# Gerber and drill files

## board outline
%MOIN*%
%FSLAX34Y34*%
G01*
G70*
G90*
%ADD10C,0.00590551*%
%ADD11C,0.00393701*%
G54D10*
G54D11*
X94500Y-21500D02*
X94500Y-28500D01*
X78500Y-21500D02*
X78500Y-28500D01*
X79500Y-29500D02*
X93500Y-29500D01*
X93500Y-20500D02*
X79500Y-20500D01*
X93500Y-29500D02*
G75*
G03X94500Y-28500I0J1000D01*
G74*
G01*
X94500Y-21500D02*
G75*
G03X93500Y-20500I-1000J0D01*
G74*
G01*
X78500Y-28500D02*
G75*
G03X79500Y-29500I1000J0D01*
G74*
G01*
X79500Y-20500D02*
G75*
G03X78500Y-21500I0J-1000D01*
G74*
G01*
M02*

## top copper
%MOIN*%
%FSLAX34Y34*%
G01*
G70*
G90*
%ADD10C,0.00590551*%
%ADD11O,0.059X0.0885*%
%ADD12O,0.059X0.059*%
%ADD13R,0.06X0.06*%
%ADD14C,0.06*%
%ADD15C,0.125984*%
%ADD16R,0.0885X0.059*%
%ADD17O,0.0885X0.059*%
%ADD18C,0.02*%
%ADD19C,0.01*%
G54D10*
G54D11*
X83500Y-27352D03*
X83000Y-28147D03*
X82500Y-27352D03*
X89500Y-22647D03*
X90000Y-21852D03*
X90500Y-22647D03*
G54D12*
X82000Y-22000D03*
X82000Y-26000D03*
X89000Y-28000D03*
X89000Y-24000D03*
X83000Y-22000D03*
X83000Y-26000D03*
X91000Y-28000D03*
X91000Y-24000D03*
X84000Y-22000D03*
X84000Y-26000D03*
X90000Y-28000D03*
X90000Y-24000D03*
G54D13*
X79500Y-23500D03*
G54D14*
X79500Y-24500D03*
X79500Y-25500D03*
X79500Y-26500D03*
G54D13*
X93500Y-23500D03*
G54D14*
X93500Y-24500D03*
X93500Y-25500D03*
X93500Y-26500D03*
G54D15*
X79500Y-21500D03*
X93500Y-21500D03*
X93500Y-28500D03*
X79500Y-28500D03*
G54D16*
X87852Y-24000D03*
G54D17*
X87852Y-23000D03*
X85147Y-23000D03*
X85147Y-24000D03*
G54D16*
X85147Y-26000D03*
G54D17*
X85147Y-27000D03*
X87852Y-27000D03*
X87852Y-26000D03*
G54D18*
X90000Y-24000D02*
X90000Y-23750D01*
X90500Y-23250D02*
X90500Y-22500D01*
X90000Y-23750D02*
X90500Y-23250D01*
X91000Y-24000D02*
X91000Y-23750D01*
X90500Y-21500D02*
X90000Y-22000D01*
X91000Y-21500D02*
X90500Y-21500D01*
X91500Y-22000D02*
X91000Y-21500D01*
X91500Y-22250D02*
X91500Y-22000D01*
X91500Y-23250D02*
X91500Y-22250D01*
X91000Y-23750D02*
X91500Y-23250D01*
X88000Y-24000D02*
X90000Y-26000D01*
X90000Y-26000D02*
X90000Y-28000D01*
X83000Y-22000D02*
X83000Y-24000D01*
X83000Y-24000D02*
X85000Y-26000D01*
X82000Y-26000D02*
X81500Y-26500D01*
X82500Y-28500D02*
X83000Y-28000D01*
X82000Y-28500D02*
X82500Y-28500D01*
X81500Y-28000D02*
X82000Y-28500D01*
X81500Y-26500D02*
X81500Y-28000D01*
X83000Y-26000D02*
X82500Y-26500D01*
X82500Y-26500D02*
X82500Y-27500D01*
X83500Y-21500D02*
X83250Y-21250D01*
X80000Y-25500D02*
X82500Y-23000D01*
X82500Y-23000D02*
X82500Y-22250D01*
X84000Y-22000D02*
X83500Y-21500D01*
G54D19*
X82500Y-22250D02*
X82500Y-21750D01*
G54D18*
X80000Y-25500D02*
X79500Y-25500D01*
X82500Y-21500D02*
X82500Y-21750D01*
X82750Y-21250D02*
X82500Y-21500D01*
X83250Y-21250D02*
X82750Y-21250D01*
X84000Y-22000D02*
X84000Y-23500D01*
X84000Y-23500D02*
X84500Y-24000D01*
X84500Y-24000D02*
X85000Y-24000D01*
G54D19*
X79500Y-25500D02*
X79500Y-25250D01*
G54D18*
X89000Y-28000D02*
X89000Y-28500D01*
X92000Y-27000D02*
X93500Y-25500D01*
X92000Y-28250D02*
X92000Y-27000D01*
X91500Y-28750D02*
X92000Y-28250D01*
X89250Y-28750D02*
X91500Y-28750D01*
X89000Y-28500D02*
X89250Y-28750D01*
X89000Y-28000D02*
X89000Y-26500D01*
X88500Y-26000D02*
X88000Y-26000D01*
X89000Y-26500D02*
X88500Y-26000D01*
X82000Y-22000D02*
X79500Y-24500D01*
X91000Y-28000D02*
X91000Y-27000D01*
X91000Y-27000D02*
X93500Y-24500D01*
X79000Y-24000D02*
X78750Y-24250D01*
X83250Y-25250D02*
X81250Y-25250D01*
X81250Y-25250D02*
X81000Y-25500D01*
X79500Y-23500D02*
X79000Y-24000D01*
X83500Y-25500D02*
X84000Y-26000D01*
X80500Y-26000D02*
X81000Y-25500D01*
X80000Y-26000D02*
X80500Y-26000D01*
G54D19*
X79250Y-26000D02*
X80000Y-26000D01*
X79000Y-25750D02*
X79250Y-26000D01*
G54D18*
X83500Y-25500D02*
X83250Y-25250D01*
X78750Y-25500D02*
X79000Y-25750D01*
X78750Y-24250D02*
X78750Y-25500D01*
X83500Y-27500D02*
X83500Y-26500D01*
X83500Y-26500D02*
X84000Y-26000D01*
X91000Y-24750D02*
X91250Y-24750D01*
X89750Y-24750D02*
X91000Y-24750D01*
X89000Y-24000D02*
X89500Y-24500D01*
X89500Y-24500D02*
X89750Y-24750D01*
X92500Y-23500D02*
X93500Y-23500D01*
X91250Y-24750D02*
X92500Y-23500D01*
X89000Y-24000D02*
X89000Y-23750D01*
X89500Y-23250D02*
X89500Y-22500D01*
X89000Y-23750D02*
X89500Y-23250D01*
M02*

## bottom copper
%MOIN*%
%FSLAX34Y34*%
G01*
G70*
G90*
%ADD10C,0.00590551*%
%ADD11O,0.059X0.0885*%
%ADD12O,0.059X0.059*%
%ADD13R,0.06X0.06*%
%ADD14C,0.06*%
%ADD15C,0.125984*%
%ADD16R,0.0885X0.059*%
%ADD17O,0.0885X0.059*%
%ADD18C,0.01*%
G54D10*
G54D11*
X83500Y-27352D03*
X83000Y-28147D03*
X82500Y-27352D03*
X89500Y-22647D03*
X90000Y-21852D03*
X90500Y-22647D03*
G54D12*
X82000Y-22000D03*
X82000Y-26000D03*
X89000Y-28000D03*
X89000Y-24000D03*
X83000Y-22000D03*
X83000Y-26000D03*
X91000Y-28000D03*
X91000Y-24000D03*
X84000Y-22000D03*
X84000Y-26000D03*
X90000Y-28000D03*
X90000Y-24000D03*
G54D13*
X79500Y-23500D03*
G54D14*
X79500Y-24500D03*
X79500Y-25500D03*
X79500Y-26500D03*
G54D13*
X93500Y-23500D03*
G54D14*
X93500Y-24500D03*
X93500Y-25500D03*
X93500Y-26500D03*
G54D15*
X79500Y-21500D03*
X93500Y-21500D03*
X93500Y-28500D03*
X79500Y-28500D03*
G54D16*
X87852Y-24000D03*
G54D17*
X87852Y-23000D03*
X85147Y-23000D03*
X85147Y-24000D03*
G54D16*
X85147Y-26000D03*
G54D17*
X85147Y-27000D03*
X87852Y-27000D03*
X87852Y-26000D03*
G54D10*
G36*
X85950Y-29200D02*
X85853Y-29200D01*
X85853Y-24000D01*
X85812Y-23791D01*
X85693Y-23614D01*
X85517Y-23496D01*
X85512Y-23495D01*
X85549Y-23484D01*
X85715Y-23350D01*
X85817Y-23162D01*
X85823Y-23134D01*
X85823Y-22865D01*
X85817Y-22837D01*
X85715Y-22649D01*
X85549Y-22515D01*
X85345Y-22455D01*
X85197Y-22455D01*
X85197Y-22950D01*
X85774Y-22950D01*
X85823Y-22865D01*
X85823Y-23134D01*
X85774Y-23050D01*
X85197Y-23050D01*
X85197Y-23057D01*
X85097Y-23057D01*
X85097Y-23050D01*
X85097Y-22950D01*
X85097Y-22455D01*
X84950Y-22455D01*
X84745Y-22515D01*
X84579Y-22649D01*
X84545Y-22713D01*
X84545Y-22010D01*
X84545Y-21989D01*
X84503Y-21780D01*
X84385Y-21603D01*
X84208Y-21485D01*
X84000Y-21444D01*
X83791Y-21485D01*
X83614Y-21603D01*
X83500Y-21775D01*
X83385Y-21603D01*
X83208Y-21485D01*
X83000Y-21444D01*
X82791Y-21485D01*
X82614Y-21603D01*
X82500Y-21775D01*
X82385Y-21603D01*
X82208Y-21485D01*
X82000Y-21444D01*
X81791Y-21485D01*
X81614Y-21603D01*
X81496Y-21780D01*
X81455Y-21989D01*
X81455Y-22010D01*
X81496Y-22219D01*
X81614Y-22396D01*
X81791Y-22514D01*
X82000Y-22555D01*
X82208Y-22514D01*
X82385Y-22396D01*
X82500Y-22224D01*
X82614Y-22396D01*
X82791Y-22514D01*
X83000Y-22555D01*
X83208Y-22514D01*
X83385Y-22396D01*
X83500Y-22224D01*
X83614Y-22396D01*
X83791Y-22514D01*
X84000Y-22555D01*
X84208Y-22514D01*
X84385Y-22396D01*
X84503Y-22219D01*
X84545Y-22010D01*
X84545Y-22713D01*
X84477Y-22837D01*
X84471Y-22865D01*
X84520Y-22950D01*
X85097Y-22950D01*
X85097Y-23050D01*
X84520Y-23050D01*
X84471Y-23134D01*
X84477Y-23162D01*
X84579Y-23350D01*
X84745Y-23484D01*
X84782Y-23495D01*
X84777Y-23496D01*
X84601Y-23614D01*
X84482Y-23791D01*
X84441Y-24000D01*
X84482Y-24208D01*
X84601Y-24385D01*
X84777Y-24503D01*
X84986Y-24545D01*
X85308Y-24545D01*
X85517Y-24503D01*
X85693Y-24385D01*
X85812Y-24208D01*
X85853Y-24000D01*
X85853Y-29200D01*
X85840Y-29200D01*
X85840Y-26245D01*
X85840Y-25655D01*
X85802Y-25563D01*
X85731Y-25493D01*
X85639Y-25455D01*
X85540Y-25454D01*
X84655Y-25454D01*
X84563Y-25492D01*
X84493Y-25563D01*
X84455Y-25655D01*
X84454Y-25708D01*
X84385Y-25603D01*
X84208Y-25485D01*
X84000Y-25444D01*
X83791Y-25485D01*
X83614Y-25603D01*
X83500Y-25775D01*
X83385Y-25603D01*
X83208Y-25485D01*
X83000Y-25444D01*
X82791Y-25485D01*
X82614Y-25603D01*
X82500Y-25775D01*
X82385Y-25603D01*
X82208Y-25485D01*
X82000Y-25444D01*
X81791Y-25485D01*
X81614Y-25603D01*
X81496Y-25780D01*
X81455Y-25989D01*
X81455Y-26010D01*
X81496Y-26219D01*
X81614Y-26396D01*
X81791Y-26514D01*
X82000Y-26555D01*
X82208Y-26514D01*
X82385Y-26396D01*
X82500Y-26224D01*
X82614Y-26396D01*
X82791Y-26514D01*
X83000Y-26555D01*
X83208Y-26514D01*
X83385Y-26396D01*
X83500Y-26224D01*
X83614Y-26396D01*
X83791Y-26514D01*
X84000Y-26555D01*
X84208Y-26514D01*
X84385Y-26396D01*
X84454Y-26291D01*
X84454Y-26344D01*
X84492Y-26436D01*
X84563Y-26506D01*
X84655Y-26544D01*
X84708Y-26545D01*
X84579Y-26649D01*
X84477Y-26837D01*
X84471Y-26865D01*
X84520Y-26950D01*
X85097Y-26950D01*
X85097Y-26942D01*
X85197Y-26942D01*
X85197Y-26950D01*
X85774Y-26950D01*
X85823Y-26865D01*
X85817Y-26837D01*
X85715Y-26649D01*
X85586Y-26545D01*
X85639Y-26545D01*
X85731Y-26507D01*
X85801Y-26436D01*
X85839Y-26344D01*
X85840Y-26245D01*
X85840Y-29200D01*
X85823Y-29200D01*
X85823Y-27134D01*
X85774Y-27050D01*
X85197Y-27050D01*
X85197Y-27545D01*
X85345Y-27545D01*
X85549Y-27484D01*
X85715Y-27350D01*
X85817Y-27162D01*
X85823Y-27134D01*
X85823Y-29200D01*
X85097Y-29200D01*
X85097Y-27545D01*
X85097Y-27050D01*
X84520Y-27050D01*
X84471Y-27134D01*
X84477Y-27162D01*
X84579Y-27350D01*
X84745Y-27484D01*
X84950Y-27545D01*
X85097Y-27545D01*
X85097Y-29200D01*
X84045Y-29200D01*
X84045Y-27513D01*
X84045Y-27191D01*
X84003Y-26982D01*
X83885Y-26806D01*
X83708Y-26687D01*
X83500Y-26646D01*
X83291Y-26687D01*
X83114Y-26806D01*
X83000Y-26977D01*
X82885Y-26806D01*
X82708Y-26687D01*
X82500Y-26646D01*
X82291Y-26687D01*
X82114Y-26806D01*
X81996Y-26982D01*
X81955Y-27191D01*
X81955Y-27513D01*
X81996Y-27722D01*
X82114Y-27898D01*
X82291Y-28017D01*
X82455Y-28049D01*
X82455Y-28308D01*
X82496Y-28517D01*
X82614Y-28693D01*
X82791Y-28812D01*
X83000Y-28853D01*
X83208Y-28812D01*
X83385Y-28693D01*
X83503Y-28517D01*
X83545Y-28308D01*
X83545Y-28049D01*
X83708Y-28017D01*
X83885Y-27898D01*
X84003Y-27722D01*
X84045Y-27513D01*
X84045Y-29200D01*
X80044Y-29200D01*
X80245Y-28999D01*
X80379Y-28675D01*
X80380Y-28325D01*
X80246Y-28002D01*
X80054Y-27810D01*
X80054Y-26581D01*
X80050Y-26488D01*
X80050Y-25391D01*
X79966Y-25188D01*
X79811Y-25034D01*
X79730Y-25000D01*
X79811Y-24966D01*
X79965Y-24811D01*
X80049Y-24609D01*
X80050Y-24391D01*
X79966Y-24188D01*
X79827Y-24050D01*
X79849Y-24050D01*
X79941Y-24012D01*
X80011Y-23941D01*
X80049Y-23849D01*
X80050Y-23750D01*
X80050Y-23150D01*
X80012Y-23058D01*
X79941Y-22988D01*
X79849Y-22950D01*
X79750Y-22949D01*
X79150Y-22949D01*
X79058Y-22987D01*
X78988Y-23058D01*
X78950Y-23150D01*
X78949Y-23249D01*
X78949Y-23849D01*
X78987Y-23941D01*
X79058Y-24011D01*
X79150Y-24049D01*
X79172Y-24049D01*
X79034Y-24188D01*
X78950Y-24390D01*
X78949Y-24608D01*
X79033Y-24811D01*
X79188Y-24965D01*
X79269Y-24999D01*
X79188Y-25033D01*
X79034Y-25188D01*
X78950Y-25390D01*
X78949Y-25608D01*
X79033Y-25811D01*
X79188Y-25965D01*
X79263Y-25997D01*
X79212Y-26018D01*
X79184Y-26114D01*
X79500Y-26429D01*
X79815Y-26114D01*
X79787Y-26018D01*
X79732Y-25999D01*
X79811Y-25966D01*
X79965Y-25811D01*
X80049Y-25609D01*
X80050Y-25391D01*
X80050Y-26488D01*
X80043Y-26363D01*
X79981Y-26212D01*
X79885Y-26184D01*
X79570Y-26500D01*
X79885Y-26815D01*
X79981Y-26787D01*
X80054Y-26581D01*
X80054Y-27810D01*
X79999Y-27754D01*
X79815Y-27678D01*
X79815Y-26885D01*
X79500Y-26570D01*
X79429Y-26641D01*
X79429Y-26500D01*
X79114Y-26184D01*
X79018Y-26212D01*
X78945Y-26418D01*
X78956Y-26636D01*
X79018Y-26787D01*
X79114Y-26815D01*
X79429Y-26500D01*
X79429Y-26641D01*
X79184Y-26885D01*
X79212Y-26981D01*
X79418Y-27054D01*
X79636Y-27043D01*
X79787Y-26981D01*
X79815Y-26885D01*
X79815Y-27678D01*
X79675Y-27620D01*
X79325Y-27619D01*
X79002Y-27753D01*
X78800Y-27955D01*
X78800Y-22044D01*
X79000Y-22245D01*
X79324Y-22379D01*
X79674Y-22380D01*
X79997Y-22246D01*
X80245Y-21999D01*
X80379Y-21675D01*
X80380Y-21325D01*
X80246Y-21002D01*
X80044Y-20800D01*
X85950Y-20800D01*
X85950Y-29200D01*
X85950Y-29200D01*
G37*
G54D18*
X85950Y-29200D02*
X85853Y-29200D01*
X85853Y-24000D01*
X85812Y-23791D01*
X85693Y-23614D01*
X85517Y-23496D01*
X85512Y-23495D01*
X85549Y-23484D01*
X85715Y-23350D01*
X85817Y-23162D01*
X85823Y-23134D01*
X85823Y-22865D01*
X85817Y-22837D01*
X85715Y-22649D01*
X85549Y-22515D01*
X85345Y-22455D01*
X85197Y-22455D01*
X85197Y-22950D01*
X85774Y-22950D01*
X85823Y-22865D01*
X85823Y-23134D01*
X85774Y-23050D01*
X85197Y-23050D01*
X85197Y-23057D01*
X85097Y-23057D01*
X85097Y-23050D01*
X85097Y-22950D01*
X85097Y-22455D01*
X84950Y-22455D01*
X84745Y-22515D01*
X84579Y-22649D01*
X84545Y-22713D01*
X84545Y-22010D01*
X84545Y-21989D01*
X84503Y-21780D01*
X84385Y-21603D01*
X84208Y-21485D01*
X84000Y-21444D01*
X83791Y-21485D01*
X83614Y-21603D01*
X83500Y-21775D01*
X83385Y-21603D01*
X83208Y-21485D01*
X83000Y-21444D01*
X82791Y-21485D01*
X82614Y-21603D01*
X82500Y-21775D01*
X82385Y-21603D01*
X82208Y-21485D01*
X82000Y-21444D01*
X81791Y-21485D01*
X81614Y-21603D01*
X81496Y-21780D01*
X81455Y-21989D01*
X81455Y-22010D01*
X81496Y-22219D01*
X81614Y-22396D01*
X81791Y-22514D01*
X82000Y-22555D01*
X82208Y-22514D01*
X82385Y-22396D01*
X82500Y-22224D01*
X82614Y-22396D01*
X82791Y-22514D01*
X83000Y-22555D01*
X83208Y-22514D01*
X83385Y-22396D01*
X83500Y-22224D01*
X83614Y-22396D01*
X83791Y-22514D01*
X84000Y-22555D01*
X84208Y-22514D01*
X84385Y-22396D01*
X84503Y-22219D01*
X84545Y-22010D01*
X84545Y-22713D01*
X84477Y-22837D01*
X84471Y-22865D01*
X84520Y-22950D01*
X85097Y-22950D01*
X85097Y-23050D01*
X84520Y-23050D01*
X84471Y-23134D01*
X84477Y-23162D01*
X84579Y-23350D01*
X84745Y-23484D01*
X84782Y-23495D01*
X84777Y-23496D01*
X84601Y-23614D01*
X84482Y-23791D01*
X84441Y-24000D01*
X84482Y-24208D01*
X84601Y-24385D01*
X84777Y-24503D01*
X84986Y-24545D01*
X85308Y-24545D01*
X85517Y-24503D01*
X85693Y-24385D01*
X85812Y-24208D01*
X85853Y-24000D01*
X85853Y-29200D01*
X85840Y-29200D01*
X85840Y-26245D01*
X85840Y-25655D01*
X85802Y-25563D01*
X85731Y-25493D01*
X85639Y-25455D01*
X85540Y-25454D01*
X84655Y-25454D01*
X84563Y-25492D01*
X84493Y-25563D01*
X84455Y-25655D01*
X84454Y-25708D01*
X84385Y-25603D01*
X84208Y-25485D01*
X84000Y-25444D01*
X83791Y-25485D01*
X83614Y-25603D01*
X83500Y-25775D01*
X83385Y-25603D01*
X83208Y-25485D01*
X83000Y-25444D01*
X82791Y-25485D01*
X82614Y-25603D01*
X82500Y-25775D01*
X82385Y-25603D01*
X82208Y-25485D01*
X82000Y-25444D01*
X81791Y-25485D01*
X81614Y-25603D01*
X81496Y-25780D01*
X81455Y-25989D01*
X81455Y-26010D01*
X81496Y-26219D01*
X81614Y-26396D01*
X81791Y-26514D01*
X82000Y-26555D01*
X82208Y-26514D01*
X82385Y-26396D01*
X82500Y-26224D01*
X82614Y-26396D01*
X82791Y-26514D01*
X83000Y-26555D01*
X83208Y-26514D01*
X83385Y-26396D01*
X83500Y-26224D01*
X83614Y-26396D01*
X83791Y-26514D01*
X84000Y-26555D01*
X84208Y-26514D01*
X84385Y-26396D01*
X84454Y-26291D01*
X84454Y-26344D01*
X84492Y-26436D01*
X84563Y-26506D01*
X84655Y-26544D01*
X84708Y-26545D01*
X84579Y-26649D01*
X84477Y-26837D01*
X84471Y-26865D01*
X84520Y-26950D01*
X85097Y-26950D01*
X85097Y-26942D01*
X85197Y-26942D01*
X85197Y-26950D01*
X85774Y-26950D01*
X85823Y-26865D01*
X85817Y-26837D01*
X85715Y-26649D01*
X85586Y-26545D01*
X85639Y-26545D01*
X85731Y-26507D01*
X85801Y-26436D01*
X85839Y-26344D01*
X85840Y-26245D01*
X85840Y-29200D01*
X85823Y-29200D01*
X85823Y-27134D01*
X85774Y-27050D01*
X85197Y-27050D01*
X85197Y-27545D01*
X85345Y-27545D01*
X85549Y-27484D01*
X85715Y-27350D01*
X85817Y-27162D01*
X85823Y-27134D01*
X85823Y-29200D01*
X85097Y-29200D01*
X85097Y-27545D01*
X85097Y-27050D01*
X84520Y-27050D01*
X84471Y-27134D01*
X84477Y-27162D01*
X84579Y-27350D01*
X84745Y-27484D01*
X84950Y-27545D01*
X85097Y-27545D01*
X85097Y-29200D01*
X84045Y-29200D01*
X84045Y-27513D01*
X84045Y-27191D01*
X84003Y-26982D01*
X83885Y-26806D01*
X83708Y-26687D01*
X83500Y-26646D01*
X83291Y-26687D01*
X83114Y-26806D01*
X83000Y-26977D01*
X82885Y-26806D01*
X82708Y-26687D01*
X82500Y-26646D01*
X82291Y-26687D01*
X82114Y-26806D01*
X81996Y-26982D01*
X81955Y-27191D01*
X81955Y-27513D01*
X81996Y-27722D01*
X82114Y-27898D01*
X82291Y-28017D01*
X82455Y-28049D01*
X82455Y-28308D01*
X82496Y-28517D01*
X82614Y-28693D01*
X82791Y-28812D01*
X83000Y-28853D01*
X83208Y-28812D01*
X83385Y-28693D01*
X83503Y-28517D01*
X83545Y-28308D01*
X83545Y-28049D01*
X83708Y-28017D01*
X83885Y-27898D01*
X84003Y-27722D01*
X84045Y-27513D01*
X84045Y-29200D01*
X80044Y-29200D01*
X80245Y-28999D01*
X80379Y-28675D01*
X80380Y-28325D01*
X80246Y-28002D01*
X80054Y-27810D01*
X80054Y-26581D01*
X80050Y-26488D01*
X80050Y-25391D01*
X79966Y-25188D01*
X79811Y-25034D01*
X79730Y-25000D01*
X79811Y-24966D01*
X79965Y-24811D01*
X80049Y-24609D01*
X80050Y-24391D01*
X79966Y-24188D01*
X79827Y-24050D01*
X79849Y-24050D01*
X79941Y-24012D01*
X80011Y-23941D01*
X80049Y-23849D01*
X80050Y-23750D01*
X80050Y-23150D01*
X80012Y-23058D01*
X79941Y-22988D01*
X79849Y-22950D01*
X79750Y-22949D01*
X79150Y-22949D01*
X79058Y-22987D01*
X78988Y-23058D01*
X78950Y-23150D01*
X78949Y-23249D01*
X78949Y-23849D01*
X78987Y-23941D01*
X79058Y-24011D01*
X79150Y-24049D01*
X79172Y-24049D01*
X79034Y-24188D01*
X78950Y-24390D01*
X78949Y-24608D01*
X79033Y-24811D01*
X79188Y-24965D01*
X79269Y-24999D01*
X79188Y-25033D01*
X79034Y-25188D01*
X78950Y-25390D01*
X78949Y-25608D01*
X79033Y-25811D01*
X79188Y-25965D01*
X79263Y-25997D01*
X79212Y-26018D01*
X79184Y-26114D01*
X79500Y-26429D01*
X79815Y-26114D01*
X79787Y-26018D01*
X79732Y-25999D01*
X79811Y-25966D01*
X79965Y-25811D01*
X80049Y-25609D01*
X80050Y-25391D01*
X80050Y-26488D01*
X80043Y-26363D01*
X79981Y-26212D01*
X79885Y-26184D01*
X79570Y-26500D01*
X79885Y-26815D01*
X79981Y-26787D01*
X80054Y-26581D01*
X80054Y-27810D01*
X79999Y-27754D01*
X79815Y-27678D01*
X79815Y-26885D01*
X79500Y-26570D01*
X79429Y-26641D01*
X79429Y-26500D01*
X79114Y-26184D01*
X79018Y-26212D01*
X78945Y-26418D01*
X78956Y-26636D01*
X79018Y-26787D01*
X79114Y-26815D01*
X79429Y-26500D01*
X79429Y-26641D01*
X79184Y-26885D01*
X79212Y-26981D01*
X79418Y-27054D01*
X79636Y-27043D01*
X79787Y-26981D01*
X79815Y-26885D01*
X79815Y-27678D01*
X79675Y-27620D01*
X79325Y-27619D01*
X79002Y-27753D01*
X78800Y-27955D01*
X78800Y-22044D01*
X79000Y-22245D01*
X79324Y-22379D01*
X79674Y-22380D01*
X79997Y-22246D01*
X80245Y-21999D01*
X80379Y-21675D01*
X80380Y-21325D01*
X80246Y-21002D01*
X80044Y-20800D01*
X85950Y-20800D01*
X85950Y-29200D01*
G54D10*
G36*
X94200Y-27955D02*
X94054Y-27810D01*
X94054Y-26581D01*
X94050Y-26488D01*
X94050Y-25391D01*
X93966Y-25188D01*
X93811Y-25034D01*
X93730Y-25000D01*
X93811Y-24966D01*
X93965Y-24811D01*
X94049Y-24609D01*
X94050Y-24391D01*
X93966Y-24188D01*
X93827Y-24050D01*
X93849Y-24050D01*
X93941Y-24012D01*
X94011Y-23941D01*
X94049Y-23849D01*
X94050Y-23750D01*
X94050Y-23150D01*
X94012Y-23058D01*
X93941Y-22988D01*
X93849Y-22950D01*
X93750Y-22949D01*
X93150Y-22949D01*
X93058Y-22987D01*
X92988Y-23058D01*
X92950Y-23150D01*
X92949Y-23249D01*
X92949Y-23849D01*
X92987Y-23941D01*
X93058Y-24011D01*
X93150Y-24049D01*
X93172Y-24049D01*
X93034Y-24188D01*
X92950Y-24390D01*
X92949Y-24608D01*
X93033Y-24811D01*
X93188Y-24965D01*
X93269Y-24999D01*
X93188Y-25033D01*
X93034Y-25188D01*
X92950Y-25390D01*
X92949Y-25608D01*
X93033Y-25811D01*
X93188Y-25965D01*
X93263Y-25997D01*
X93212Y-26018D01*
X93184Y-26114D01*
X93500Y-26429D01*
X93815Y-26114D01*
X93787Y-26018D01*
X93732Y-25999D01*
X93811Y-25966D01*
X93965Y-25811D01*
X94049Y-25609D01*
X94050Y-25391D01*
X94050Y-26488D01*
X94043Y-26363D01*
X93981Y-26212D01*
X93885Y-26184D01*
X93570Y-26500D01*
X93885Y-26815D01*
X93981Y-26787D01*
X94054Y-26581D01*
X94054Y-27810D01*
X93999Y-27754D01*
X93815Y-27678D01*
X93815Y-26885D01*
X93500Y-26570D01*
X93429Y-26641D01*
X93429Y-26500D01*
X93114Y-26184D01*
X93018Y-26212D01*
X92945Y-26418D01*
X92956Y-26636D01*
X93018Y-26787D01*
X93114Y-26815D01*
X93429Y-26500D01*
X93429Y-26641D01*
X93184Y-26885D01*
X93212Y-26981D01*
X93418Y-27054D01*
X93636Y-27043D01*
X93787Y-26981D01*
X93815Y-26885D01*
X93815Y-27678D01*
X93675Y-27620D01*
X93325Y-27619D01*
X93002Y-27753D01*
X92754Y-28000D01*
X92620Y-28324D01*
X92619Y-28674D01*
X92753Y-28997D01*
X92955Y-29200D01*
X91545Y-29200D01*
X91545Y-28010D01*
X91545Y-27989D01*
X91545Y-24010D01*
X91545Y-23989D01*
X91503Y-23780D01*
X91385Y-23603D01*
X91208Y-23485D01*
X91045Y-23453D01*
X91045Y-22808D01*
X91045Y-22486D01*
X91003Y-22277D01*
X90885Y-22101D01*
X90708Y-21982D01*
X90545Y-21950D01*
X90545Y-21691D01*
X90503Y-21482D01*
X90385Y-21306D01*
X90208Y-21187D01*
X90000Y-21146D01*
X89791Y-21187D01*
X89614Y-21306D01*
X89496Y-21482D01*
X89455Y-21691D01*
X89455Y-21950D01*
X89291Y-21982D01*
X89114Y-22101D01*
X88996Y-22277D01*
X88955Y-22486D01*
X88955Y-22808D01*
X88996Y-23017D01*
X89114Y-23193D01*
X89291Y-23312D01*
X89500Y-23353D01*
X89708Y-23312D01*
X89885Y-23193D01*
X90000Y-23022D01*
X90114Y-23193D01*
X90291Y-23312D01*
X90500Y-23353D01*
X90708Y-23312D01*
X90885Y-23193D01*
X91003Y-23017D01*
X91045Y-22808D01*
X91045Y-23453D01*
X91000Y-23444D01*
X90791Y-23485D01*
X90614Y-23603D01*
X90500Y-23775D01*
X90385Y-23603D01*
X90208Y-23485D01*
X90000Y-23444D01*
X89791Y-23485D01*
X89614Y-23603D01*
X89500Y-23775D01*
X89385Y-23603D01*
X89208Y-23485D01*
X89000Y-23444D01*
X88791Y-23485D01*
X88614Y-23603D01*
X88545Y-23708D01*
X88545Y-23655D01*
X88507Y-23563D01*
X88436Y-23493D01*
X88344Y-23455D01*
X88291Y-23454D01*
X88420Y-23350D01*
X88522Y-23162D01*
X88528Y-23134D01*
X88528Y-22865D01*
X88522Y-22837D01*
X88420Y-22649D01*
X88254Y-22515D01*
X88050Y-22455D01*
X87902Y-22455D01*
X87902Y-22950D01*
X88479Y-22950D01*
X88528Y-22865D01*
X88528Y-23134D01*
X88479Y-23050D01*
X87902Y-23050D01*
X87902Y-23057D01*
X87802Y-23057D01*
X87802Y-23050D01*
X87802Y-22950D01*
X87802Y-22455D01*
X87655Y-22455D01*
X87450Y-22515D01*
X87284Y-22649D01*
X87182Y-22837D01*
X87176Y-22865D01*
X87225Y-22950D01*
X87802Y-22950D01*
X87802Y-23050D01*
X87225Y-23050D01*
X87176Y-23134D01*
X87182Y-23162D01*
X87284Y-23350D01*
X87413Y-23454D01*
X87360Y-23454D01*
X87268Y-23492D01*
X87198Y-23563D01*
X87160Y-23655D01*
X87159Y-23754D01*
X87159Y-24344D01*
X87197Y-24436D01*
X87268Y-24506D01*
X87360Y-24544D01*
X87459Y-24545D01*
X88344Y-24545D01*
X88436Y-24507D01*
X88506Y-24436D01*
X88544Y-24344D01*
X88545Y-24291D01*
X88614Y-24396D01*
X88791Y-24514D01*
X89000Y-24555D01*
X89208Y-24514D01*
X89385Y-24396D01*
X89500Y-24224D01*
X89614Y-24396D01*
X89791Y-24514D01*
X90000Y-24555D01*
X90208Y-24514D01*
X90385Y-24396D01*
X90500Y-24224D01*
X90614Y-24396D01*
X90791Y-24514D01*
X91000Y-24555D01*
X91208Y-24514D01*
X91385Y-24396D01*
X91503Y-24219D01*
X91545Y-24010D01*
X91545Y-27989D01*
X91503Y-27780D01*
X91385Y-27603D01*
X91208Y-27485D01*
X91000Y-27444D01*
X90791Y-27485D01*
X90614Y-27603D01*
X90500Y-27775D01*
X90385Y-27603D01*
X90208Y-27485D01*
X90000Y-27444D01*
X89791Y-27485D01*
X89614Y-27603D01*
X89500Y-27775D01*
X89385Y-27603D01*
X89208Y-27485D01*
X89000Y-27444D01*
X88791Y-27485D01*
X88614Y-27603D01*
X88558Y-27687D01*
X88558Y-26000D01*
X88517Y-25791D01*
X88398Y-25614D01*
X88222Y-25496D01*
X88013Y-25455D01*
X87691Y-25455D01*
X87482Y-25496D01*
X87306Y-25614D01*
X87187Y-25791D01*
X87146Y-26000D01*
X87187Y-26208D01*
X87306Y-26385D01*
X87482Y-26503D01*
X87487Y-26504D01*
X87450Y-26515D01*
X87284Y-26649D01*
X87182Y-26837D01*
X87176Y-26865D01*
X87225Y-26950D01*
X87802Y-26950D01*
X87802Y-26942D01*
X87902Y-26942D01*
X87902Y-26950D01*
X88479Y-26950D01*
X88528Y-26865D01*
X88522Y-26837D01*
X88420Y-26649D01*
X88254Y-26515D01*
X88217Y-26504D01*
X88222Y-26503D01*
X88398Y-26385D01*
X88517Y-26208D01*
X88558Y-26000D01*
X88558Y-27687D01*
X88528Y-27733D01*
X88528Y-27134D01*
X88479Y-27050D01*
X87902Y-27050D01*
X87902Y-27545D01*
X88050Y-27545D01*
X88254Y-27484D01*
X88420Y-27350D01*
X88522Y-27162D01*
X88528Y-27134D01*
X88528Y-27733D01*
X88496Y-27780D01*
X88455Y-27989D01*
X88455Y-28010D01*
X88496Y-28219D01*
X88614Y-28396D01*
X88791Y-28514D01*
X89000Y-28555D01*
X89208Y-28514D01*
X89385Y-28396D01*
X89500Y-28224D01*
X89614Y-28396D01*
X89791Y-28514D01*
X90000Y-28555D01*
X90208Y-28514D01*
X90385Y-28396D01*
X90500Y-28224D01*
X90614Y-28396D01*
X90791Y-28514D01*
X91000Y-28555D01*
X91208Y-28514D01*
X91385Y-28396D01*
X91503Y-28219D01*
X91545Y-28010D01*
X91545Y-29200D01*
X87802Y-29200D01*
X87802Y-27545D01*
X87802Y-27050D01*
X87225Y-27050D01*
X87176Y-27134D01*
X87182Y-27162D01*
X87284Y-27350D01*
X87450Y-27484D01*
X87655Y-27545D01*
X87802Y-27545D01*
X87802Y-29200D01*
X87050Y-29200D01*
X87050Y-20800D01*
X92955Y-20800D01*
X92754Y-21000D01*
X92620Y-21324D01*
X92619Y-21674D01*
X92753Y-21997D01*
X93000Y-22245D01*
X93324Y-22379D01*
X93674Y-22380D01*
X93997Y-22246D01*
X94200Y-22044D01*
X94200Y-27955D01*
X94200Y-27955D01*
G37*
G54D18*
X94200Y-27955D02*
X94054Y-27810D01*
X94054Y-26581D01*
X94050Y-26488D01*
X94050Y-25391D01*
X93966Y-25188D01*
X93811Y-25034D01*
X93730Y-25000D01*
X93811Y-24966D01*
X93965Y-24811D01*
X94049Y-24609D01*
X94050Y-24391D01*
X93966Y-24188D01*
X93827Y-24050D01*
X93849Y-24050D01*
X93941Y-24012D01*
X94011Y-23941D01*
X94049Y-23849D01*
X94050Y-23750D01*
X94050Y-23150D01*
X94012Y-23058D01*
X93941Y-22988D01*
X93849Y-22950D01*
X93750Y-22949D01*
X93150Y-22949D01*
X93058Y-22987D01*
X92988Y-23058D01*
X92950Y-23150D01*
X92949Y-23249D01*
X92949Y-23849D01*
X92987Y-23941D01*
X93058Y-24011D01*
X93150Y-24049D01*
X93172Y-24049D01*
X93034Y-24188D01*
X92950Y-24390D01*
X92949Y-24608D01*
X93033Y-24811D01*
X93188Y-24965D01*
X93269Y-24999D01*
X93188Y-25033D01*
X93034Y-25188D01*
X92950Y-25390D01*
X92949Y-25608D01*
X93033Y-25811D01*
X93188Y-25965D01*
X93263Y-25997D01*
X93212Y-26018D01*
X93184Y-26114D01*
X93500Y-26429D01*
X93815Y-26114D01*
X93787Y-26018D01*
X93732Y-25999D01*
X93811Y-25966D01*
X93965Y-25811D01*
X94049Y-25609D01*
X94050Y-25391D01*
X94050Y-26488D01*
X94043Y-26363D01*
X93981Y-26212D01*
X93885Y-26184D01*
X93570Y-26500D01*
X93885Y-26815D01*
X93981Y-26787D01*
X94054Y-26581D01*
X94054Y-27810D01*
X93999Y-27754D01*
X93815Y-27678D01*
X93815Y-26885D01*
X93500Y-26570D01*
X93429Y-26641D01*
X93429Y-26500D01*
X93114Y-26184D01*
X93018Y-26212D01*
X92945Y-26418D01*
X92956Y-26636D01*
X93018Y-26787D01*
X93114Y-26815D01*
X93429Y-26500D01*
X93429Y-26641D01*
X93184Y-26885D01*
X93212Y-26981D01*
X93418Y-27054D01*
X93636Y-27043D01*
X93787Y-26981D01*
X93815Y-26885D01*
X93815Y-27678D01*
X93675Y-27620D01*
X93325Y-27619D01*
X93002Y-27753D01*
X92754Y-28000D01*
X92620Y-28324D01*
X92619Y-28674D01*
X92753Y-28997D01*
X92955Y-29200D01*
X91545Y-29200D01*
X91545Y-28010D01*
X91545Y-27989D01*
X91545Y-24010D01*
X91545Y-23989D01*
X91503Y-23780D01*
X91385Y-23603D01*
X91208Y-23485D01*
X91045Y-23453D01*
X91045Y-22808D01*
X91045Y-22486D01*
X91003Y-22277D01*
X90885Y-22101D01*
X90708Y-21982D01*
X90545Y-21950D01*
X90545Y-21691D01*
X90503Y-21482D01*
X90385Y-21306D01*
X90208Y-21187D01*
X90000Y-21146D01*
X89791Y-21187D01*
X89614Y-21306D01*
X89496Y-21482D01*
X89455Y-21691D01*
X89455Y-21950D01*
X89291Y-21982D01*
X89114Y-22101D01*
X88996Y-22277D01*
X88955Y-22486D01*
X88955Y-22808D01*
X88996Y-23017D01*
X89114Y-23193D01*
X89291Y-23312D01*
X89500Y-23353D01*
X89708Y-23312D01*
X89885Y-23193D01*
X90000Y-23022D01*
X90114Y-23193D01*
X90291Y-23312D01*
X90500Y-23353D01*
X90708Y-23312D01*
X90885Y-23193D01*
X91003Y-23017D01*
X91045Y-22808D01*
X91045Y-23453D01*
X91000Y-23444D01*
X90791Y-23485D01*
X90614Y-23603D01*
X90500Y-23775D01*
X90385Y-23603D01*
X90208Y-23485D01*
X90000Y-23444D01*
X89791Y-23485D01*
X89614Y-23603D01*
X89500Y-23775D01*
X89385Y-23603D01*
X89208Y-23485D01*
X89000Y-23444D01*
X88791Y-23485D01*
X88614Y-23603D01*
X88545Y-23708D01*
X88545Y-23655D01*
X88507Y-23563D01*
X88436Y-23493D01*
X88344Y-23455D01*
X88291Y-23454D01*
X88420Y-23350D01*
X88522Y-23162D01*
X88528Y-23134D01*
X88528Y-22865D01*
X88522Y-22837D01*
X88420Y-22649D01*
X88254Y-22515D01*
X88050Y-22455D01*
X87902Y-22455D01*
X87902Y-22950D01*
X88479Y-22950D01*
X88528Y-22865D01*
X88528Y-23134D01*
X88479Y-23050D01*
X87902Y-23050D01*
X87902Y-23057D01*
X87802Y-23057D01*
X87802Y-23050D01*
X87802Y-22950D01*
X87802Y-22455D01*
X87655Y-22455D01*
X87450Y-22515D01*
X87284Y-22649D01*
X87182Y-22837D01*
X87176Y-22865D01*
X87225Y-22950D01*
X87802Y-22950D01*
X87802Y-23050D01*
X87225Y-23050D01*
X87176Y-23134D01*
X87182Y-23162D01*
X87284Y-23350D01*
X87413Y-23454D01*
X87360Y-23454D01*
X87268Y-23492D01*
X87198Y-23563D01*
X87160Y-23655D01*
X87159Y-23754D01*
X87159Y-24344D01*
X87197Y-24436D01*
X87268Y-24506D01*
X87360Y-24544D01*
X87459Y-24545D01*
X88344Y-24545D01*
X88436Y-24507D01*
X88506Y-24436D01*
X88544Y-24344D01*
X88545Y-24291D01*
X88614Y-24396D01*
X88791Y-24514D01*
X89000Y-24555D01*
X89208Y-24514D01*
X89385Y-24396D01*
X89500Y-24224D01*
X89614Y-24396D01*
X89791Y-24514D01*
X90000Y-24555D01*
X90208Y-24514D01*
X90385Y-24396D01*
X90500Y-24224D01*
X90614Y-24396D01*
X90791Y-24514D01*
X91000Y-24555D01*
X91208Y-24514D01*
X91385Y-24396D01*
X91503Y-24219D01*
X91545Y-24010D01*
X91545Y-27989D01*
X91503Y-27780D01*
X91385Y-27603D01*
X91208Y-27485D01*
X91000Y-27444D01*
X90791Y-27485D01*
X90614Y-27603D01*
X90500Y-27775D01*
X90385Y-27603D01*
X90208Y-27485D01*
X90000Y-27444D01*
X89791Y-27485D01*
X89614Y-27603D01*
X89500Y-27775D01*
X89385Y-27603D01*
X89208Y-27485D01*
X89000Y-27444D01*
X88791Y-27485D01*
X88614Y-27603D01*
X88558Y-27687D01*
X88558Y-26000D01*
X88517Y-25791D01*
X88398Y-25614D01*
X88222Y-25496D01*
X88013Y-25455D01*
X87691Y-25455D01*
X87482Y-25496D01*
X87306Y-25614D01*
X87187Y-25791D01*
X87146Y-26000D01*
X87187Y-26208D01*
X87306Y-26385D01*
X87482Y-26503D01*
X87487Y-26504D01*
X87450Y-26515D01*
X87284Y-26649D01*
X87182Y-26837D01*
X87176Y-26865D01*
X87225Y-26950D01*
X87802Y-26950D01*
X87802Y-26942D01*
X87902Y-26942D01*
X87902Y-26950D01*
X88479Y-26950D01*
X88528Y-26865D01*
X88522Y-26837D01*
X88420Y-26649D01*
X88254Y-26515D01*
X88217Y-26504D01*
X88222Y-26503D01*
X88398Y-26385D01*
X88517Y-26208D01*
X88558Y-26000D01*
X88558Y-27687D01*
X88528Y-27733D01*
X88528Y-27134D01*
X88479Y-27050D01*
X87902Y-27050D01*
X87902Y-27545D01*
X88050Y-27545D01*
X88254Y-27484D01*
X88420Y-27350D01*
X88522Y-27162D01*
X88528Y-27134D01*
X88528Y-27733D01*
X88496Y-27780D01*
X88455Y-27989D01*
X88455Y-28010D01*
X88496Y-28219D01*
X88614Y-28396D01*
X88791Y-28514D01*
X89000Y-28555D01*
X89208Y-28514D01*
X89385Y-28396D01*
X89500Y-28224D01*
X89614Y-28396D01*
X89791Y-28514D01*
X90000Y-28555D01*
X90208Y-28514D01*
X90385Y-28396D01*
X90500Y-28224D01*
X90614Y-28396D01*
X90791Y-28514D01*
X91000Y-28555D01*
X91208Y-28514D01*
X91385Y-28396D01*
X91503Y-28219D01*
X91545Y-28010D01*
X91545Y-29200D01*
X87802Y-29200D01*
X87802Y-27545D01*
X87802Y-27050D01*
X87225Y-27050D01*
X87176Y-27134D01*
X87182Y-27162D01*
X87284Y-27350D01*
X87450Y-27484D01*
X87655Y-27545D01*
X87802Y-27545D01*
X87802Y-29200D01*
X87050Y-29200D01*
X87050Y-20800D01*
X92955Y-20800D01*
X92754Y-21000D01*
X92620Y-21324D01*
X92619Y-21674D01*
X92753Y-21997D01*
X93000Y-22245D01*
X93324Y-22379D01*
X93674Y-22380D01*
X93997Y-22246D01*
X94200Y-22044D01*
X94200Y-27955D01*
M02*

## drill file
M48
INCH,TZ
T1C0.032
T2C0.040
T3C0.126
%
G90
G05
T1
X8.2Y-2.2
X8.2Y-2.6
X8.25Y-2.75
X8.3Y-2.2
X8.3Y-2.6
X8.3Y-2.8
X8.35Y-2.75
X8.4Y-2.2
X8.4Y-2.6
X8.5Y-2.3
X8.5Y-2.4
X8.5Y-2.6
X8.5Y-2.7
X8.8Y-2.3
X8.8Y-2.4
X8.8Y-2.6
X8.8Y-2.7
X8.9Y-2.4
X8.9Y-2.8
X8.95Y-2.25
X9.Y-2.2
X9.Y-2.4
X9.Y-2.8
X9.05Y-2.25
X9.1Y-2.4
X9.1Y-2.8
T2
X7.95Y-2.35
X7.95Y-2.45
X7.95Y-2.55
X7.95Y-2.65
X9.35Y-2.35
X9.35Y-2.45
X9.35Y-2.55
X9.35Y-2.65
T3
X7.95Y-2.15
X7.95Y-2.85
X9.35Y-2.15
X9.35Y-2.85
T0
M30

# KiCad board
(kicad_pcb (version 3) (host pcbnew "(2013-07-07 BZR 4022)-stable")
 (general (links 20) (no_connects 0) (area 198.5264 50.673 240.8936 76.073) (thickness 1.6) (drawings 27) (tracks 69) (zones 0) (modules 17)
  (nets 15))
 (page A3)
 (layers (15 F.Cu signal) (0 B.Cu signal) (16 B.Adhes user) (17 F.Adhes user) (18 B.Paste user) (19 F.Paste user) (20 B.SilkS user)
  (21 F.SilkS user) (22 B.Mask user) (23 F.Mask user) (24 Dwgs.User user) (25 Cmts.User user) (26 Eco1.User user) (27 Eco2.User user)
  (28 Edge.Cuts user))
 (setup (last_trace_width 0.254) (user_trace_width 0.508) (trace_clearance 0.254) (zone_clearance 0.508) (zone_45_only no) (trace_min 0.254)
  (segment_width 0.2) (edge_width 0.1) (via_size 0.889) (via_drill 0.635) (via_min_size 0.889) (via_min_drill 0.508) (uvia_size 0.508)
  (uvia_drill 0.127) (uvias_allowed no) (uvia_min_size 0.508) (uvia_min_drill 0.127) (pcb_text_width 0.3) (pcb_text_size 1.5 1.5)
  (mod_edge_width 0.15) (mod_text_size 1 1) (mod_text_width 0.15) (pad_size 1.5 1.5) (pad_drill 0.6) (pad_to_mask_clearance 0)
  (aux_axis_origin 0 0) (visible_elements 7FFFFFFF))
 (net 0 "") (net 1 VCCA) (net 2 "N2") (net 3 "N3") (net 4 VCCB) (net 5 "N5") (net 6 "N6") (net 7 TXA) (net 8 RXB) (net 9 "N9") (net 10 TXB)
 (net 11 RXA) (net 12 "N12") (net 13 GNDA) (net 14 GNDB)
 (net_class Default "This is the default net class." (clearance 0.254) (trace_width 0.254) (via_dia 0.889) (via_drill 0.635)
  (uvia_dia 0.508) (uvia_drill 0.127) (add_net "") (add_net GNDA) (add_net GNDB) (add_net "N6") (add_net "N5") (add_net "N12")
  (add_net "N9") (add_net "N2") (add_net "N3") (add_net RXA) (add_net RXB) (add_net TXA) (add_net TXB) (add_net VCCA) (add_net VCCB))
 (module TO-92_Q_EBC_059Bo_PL (layer F.Cu) (at 212.09 69.85)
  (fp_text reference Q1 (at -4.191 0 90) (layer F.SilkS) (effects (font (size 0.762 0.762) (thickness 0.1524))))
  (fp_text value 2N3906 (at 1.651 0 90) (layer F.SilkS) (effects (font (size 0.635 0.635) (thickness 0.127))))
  (pad 1 thru_hole oval (at 0 0) (size 1.4986 2.2479) (drill 0.8128 (offset 0 -0.37465)) (layers *.Cu *.Mask F.SilkS) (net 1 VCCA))
  (pad 2 thru_hole oval (at -1.27 1.27) (size 1.4986 2.2479) (drill 0.8128 (offset 0 0.37465)) (layers *.Cu *.Mask F.SilkS) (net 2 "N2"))
  (pad 3 thru_hole oval (at -2.54 0) (size 1.4986 2.2479) (drill 0.8128 (offset 0 -0.37465)) (layers *.Cu *.Mask F.SilkS) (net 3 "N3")))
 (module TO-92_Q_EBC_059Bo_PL (layer F.Cu) (at 227.33 57.15 180)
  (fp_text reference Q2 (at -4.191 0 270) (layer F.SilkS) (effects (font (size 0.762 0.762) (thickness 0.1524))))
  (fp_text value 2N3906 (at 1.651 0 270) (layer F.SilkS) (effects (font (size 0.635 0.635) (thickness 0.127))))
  (pad 1 thru_hole oval (at 0 0 180) (size 1.4986 2.2479) (drill 0.8128 (offset 0 -0.37465)) (layers *.Cu *.Mask F.SilkS) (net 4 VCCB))
  (pad 2 thru_hole oval (at -1.27 1.27 180) (size 1.4986 2.2479) (drill 0.8128 (offset 0 0.37465)) (layers *.Cu *.Mask F.SilkS) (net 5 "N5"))
  (pad 3 thru_hole oval (at -2.54 0 180) (size 1.4986 2.2479) (drill 0.8128 (offset 0 -0.37465)) (layers *.Cu *.Mask F.SilkS) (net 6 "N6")))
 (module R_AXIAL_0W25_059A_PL (layer F.Cu) (at 208.28 55.88 270) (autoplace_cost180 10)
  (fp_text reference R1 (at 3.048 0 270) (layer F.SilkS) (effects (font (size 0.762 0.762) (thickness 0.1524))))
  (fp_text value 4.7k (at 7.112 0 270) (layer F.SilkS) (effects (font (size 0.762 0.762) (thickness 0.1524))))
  (pad 1 thru_hole oval (at 0 0 270) (size 1.4986 1.4986) (drill 0.8128) (layers *.Cu *.Mask F.SilkS) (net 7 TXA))
  (pad 2 thru_hole oval (at 10.16 0 270) (size 1.4986 1.4986) (drill 0.8128) (layers *.Cu *.Mask F.SilkS) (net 2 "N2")))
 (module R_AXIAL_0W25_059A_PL (layer F.Cu) (at 226.06 71.12 90) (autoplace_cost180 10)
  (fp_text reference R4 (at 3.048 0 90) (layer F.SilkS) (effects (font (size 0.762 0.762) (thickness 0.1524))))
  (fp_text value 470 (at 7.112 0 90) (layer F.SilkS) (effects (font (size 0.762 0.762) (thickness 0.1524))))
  (pad 1 thru_hole oval (at 0 0 90) (size 1.4986 1.4986) (drill 0.8128) (layers *.Cu *.Mask F.SilkS) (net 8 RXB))
  (pad 2 thru_hole oval (at 10.16 0 90) (size 1.4986 1.4986) (drill 0.8128) (layers *.Cu *.Mask F.SilkS) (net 4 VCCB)))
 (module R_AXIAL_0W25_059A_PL (layer F.Cu) (at 210.82 55.88 270) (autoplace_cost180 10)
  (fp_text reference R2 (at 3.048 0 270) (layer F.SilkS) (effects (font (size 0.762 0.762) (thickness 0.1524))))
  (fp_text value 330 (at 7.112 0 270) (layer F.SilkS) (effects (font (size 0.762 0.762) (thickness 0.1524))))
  (pad 1 thru_hole oval (at 0 0 270) (size 1.4986 1.4986) (drill 0.8128) (layers *.Cu *.Mask F.SilkS) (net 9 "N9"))
  (pad 2 thru_hole oval (at 10.16 0 270) (size 1.4986 1.4986) (drill 0.8128) (layers *.Cu *.Mask F.SilkS) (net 3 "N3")))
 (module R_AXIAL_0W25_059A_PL (layer F.Cu) (at 231.14 71.12 90) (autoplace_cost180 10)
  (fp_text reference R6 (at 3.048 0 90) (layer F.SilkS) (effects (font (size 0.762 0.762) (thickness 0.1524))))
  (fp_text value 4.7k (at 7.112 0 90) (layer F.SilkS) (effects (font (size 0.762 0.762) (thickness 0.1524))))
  (pad 1 thru_hole oval (at 0 0 90) (size 1.4986 1.4986) (drill 0.8128) (layers *.Cu *.Mask F.SilkS) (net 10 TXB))
  (pad 2 thru_hole oval (at 10.16 0 90) (size 1.4986 1.4986) (drill 0.8128) (layers *.Cu *.Mask F.SilkS) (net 5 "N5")))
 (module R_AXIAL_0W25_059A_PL (layer F.Cu) (at 213.36 55.88 270) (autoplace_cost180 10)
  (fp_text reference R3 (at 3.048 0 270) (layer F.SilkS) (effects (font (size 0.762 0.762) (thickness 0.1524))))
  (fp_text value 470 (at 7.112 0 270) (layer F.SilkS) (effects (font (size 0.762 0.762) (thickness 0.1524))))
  (pad 1 thru_hole oval (at 0 0 270) (size 1.4986 1.4986) (drill 0.8128) (layers *.Cu *.Mask F.SilkS) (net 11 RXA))
  (pad 2 thru_hole oval (at 10.16 0 270) (size 1.4986 1.4986) (drill 0.8128) (layers *.Cu *.Mask F.SilkS) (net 1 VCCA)))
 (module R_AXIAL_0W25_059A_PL (layer F.Cu) (at 228.6 71.12 90) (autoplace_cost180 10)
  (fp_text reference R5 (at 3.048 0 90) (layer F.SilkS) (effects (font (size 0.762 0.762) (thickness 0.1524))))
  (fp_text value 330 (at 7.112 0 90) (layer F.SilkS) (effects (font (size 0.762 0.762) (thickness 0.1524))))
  (pad 1 thru_hole oval (at 0 0 90) (size 1.4986 1.4986) (drill 0.8128) (layers *.Cu *.Mask F.SilkS) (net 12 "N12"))
  (pad 2 thru_hole oval (at 10.16 0 90) (size 1.4986 1.4986) (drill 0.8128) (layers *.Cu *.Mask F.SilkS) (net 6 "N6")))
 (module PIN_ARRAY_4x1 (layer F.Cu) (at 201.93 63.5 270)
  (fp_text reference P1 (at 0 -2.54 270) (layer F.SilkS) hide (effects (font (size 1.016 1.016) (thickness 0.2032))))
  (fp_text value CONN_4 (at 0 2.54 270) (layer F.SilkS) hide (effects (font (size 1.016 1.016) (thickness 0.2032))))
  (pad 1 thru_hole rect (at -3.81 0 270) (size 1.524 1.524) (drill 1.016) (layers *.Cu *.Mask F.SilkS) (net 1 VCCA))
  (pad 2 thru_hole circle (at -1.27 0 270) (size 1.524 1.524) (drill 1.016) (layers *.Cu *.Mask F.SilkS) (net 7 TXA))
  (pad 3 thru_hole circle (at 1.27 0 270) (size 1.524 1.524) (drill 1.016) (layers *.Cu *.Mask F.SilkS) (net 11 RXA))
  (pad 4 thru_hole circle (at 3.81 0 270) (size 1.524 1.524) (drill 1.016) (layers *.Cu *.Mask F.SilkS) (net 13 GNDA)))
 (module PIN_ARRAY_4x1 (layer F.Cu) (at 237.49 63.5 270)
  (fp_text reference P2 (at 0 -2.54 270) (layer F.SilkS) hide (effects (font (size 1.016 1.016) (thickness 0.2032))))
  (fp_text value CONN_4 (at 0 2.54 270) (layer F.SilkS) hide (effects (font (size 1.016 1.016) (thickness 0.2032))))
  (pad 1 thru_hole rect (at -3.81 0 270) (size 1.524 1.524) (drill 1.016) (layers *.Cu *.Mask F.SilkS) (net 4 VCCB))
  (pad 2 thru_hole circle (at -1.27 0 270) (size 1.524 1.524) (drill 1.016) (layers *.Cu *.Mask F.SilkS) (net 10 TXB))
  (pad 3 thru_hole circle (at 1.27 0 270) (size 1.524 1.524) (drill 1.016) (layers *.Cu *.Mask F.SilkS) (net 8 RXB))
  (pad 4 thru_hole circle (at 3.81 0 270) (size 1.524 1.524) (drill 1.016) (layers *.Cu *.Mask F.SilkS) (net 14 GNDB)))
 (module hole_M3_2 (layer F.Cu) (at 201.93 54.61)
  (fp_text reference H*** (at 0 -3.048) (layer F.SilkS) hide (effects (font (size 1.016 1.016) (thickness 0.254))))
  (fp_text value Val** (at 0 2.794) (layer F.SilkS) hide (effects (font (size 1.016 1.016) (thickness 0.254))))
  (pad 1 thru_hole circle (at 0 0) (size 3.2 3.2) (drill 3.2) (layers *.Cu *.Mask F.SilkS)))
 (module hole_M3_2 (layer F.Cu) (at 237.49 54.61)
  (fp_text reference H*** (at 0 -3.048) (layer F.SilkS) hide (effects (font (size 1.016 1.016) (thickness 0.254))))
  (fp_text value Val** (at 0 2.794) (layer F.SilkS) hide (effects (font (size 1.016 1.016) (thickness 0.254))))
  (pad 1 thru_hole circle (at 0 0) (size 3.2 3.2) (drill 3.2) (layers *.Cu *.Mask F.SilkS)))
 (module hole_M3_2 (layer F.Cu) (at 237.49 72.39)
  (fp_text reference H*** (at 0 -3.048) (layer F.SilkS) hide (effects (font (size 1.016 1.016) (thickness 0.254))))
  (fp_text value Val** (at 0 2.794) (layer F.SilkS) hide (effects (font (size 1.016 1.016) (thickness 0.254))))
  (pad 1 thru_hole circle (at 0 0) (size 3.2 3.2) (drill 3.2) (layers *.Cu *.Mask F.SilkS)))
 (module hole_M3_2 (layer F.Cu) (at 201.93 72.39)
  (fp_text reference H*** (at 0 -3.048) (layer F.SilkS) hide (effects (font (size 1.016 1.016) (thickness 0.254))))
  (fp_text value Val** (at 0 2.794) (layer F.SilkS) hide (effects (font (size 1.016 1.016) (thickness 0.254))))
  (pad 1 thru_hole circle (at 0 0) (size 3.2 3.2) (drill 3.2) (layers *.Cu *.Mask F.SilkS)))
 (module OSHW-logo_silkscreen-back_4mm (layer F.Cu) (at 210.82 60.325)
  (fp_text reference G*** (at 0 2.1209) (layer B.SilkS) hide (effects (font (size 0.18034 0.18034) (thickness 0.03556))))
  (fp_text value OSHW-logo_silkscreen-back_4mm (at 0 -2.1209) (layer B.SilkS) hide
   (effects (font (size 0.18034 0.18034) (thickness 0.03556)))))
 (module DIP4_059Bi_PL (layer F.Cu) (at 219.71 59.69 90)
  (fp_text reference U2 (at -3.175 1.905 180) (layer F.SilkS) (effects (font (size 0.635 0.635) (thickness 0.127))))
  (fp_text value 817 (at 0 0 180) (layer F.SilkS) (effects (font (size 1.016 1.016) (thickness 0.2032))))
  (pad 1 thru_hole rect (at -1.27 3.81 90) (size 1.4986 2.2479) (drill 0.8128 (offset 0 -0.37465)) (layers *.Cu *.Mask F.SilkS)
   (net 12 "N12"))
  (pad 2 thru_hole oval (at 1.27 3.81 90) (size 1.4986 2.2479) (drill 0.8128 (offset 0 -0.37465)) (layers *.Cu *.Mask F.SilkS) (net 14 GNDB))
  (pad 3 thru_hole oval (at 1.27 -3.81 90) (size 1.4986 2.2479) (drill 0.8128 (offset 0 0.37465)) (layers *.Cu *.Mask F.SilkS) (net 13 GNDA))
  (pad 4 thru_hole oval (at -1.27 -3.81 90) (size 1.4986 2.2479) (drill 0.8128 (offset 0 0.37465)) (layers *.Cu *.Mask F.SilkS) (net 11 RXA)))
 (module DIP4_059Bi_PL (layer F.Cu) (at 219.71 67.31 270)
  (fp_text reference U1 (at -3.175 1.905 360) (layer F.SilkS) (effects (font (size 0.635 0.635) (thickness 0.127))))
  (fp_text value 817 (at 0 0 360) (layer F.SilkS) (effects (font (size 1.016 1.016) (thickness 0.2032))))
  (pad 1 thru_hole rect (at -1.27 3.81 270) (size 1.4986 2.2479) (drill 0.8128 (offset 0 -0.37465)) (layers *.Cu *.Mask F.SilkS)
   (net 9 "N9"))
  (pad 2 thru_hole oval (at 1.27 3.81 270) (size 1.4986 2.2479) (drill 0.8128 (offset 0 -0.37465)) (layers *.Cu *.Mask F.SilkS)
   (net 13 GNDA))
  (pad 3 thru_hole oval (at 1.27 -3.81 270) (size 1.4986 2.2479) (drill 0.8128 (offset 0 0.37465)) (layers *.Cu *.Mask F.SilkS)
   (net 14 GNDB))
  (pad 4 thru_hole oval (at -1.27 -3.81 270) (size 1.4986 2.2479) (drill 0.8128 (offset 0 0.37465)) (layers *.Cu *.Mask F.SilkS) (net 8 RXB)))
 (gr_line (start 240.03 54.61) (end 240.03 72.39) (angle 90) (layer Edge.Cuts) (width 0.1))
 (gr_line (start 199.39 54.61) (end 199.39 72.39) (angle 90) (layer Edge.Cuts) (width 0.1))
 (gr_line (start 201.93 74.93) (end 237.49 74.93) (angle 90) (layer Edge.Cuts) (width 0.1))
 (gr_line (start 237.49 52.07) (end 201.93 52.07) (angle 90) (layer Edge.Cuts) (width 0.1))
 (gr_arc (start 237.49 72.39) (end 240.03 72.39) (angle 90) (layer Edge.Cuts) (width 0.1))
 (gr_arc (start 237.49 54.61) (end 237.49 52.07) (angle 90) (layer Edge.Cuts) (width 0.1))
 (gr_arc (start 201.93 72.39) (end 201.93 74.93) (angle 90) (layer Edge.Cuts) (width 0.1))
 (gr_arc (start 201.93 54.61) (end 199.39 54.61) (angle 90) (layer Edge.Cuts) (width 0.1))
 (segment (start 228.6 60.96) (end 228.6 60.325) (width 0.508) (layer F.Cu) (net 6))
 (segment (start 229.87 59.055) (end 229.87 57.15) (width 0.508) (layer F.Cu) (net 6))
 (segment (start 228.6 60.325) (end 229.87 59.055) (width 0.508) (layer F.Cu) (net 6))
 (segment (start 231.14 60.96) (end 231.14 60.325) (width 0.508) (layer F.Cu) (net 5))
 (segment (start 229.87 54.61) (end 228.6 55.88) (width 0.508) (layer F.Cu) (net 5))
 (segment (start 231.14 54.61) (end 229.87 54.61) (width 0.508) (layer F.Cu) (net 5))
 (segment (start 232.41 55.88) (end 231.14 54.61) (width 0.508) (layer F.Cu) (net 5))
 (segment (start 232.41 56.515) (end 232.41 55.88) (width 0.508) (layer F.Cu) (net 5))
 (segment (start 232.41 59.055) (end 232.41 56.515) (width 0.508) (layer F.Cu) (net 5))
 (segment (start 231.14 60.325) (end 232.41 59.055) (width 0.508) (layer F.Cu) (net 5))
 (segment (start 223.52 60.96) (end 228.6 66.04) (width 0.508) (layer F.Cu) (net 12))
 (segment (start 228.6 66.04) (end 228.6 71.12) (width 0.508) (layer F.Cu) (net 12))
 (segment (start 210.82 55.88) (end 210.82 60.96) (width 0.508) (layer F.Cu) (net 9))
 (segment (start 210.82 60.96) (end 215.9 66.04) (width 0.508) (layer F.Cu) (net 9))
 (segment (start 208.28 66.04) (end 207.01 67.31) (width 0.508) (layer F.Cu) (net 2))
 (segment (start 209.55 72.39) (end 210.82 71.12) (width 0.508) (layer F.Cu) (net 2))
 (segment (start 208.28 72.39) (end 209.55 72.39) (width 0.508) (layer F.Cu) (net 2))
 (segment (start 207.01 71.12) (end 208.28 72.39) (width 0.508) (layer F.Cu) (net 2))
 (segment (start 207.01 67.31) (end 207.01 71.12) (width 0.508) (layer F.Cu) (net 2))
 (segment (start 210.82 66.04) (end 209.55 67.31) (width 0.508) (layer F.Cu) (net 3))
 (segment (start 209.55 67.31) (end 209.55 69.85) (width 0.508) (layer F.Cu) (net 3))
 (segment (start 212.09 54.61) (end 211.455 53.975) (width 0.508) (layer F.Cu) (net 11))
 (segment (start 203.2 64.77) (end 209.55 58.42) (width 0.508) (layer F.Cu) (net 11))
 (segment (start 209.55 58.42) (end 209.55 56.515) (width 0.508) (layer F.Cu) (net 11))
 (segment (start 213.36 55.88) (end 212.09 54.61) (width 0.508) (layer F.Cu) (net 11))
 (segment (start 209.55 56.515) (end 209.55 55.245) (width 0.254) (layer F.Cu) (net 11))
 (segment (start 203.2 64.77) (end 201.93 64.77) (width 0.508) (layer F.Cu) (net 11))
 (segment (start 209.55 54.61) (end 209.55 55.245) (width 0.508) (layer F.Cu) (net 11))
 (segment (start 210.185 53.975) (end 209.55 54.61) (width 0.508) (layer F.Cu) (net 11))
 (segment (start 211.455 53.975) (end 210.185 53.975) (width 0.508) (layer F.Cu) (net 11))
 (segment (start 213.36 55.88) (end 213.36 59.69) (width 0.508) (layer F.Cu) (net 11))
 (segment (start 213.36 59.69) (end 214.63 60.96) (width 0.508) (layer F.Cu) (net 11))
 (segment (start 214.63 60.96) (end 215.9 60.96) (width 0.508) (layer F.Cu) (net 11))
 (segment (start 201.93 64.77) (end 201.93 64.135) (width 0.254) (layer F.Cu) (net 11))
 (segment (start 226.06 71.12) (end 226.06 72.39) (width 0.508) (layer F.Cu) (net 8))
 (segment (start 233.68 68.58) (end 237.49 64.77) (width 0.508) (layer F.Cu) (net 8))
 (segment (start 233.68 71.755) (end 233.68 68.58) (width 0.508) (layer F.Cu) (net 8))
 (segment (start 232.41 73.025) (end 233.68 71.755) (width 0.508) (layer F.Cu) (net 8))
 (segment (start 226.695 73.025) (end 232.41 73.025) (width 0.508) (layer F.Cu) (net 8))
 (segment (start 226.06 72.39) (end 226.695 73.025) (width 0.508) (layer F.Cu) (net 8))
 (segment (start 226.06 71.12) (end 226.06 67.31) (width 0.508) (layer F.Cu) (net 8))
 (segment (start 224.79 66.04) (end 223.52 66.04) (width 0.508) (layer F.Cu) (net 8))
 (segment (start 226.06 67.31) (end 224.79 66.04) (width 0.508) (layer F.Cu) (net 8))
 (segment (start 208.28 55.88) (end 201.93 62.23) (width 0.508) (layer F.Cu) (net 7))
 (segment (start 231.14 71.12) (end 231.14 68.58) (width 0.508) (layer F.Cu) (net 10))
 (segment (start 231.14 68.58) (end 237.49 62.23) (width 0.508) (layer F.Cu) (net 10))
 (segment (start 200.66 60.96) (end 200.025 61.595) (width 0.508) (layer F.Cu) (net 1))
 (segment (start 211.455 64.135) (end 206.375 64.135) (width 0.508) (layer F.Cu) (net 1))
 (segment (start 206.375 64.135) (end 205.74 64.77) (width 0.508) (layer F.Cu) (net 1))
 (segment (start 201.93 59.69) (end 200.66 60.96) (width 0.508) (layer F.Cu) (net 1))
 (segment (start 212.09 64.77) (end 213.36 66.04) (width 0.508) (layer F.Cu) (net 1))
 (segment (start 204.47 66.04) (end 205.74 64.77) (width 0.508) (layer F.Cu) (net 1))
 (segment (start 203.2 66.04) (end 204.47 66.04) (width 0.508) (layer F.Cu) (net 1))
 (segment (start 201.295 66.04) (end 203.2 66.04) (width 0.254) (layer F.Cu) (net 1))
 (segment (start 200.66 65.405) (end 201.295 66.04) (width 0.254) (layer F.Cu) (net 1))
 (segment (start 212.09 64.77) (end 211.455 64.135) (width 0.508) (layer F.Cu) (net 1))
 (segment (start 200.025 64.77) (end 200.66 65.405) (width 0.508) (layer F.Cu) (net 1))
 (segment (start 200.025 61.595) (end 200.025 64.77) (width 0.508) (layer F.Cu) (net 1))
 (segment (start 212.09 69.85) (end 212.09 67.31) (width 0.508) (layer F.Cu) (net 1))
 (segment (start 212.09 67.31) (end 213.36 66.04) (width 0.508) (layer F.Cu) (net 1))
 (segment (start 231.14 62.865) (end 231.775 62.865) (width 0.508) (layer F.Cu) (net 4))
 (segment (start 227.965 62.865) (end 231.14 62.865) (width 0.508) (layer F.Cu) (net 4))
 (segment (start 226.06 60.96) (end 227.33 62.23) (width 0.508) (layer F.Cu) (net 4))
 (segment (start 227.33 62.23) (end 227.965 62.865) (width 0.508) (layer F.Cu) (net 4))
 (segment (start 234.95 59.69) (end 237.49 59.69) (width 0.508) (layer F.Cu) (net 4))
 (segment (start 231.775 62.865) (end 234.95 59.69) (width 0.508) (layer F.Cu) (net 4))
 (segment (start 226.06 60.96) (end 226.06 60.325) (width 0.508) (layer F.Cu) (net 4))
 (segment (start 227.33 59.055) (end 227.33 57.15) (width 0.508) (layer F.Cu) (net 4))
 (segment (start 226.06 60.325) (end 227.33 59.055) (width 0.508) (layer F.Cu) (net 4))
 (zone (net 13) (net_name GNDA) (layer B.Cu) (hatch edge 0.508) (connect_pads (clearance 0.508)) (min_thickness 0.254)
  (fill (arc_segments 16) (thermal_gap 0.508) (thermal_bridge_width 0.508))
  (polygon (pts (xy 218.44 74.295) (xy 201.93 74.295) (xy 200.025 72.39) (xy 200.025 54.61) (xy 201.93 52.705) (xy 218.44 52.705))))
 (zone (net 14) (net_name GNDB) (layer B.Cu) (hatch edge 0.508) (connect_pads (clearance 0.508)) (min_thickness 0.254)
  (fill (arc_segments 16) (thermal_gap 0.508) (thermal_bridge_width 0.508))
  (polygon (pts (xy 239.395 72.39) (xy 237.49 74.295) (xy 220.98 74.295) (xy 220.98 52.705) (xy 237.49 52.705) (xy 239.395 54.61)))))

